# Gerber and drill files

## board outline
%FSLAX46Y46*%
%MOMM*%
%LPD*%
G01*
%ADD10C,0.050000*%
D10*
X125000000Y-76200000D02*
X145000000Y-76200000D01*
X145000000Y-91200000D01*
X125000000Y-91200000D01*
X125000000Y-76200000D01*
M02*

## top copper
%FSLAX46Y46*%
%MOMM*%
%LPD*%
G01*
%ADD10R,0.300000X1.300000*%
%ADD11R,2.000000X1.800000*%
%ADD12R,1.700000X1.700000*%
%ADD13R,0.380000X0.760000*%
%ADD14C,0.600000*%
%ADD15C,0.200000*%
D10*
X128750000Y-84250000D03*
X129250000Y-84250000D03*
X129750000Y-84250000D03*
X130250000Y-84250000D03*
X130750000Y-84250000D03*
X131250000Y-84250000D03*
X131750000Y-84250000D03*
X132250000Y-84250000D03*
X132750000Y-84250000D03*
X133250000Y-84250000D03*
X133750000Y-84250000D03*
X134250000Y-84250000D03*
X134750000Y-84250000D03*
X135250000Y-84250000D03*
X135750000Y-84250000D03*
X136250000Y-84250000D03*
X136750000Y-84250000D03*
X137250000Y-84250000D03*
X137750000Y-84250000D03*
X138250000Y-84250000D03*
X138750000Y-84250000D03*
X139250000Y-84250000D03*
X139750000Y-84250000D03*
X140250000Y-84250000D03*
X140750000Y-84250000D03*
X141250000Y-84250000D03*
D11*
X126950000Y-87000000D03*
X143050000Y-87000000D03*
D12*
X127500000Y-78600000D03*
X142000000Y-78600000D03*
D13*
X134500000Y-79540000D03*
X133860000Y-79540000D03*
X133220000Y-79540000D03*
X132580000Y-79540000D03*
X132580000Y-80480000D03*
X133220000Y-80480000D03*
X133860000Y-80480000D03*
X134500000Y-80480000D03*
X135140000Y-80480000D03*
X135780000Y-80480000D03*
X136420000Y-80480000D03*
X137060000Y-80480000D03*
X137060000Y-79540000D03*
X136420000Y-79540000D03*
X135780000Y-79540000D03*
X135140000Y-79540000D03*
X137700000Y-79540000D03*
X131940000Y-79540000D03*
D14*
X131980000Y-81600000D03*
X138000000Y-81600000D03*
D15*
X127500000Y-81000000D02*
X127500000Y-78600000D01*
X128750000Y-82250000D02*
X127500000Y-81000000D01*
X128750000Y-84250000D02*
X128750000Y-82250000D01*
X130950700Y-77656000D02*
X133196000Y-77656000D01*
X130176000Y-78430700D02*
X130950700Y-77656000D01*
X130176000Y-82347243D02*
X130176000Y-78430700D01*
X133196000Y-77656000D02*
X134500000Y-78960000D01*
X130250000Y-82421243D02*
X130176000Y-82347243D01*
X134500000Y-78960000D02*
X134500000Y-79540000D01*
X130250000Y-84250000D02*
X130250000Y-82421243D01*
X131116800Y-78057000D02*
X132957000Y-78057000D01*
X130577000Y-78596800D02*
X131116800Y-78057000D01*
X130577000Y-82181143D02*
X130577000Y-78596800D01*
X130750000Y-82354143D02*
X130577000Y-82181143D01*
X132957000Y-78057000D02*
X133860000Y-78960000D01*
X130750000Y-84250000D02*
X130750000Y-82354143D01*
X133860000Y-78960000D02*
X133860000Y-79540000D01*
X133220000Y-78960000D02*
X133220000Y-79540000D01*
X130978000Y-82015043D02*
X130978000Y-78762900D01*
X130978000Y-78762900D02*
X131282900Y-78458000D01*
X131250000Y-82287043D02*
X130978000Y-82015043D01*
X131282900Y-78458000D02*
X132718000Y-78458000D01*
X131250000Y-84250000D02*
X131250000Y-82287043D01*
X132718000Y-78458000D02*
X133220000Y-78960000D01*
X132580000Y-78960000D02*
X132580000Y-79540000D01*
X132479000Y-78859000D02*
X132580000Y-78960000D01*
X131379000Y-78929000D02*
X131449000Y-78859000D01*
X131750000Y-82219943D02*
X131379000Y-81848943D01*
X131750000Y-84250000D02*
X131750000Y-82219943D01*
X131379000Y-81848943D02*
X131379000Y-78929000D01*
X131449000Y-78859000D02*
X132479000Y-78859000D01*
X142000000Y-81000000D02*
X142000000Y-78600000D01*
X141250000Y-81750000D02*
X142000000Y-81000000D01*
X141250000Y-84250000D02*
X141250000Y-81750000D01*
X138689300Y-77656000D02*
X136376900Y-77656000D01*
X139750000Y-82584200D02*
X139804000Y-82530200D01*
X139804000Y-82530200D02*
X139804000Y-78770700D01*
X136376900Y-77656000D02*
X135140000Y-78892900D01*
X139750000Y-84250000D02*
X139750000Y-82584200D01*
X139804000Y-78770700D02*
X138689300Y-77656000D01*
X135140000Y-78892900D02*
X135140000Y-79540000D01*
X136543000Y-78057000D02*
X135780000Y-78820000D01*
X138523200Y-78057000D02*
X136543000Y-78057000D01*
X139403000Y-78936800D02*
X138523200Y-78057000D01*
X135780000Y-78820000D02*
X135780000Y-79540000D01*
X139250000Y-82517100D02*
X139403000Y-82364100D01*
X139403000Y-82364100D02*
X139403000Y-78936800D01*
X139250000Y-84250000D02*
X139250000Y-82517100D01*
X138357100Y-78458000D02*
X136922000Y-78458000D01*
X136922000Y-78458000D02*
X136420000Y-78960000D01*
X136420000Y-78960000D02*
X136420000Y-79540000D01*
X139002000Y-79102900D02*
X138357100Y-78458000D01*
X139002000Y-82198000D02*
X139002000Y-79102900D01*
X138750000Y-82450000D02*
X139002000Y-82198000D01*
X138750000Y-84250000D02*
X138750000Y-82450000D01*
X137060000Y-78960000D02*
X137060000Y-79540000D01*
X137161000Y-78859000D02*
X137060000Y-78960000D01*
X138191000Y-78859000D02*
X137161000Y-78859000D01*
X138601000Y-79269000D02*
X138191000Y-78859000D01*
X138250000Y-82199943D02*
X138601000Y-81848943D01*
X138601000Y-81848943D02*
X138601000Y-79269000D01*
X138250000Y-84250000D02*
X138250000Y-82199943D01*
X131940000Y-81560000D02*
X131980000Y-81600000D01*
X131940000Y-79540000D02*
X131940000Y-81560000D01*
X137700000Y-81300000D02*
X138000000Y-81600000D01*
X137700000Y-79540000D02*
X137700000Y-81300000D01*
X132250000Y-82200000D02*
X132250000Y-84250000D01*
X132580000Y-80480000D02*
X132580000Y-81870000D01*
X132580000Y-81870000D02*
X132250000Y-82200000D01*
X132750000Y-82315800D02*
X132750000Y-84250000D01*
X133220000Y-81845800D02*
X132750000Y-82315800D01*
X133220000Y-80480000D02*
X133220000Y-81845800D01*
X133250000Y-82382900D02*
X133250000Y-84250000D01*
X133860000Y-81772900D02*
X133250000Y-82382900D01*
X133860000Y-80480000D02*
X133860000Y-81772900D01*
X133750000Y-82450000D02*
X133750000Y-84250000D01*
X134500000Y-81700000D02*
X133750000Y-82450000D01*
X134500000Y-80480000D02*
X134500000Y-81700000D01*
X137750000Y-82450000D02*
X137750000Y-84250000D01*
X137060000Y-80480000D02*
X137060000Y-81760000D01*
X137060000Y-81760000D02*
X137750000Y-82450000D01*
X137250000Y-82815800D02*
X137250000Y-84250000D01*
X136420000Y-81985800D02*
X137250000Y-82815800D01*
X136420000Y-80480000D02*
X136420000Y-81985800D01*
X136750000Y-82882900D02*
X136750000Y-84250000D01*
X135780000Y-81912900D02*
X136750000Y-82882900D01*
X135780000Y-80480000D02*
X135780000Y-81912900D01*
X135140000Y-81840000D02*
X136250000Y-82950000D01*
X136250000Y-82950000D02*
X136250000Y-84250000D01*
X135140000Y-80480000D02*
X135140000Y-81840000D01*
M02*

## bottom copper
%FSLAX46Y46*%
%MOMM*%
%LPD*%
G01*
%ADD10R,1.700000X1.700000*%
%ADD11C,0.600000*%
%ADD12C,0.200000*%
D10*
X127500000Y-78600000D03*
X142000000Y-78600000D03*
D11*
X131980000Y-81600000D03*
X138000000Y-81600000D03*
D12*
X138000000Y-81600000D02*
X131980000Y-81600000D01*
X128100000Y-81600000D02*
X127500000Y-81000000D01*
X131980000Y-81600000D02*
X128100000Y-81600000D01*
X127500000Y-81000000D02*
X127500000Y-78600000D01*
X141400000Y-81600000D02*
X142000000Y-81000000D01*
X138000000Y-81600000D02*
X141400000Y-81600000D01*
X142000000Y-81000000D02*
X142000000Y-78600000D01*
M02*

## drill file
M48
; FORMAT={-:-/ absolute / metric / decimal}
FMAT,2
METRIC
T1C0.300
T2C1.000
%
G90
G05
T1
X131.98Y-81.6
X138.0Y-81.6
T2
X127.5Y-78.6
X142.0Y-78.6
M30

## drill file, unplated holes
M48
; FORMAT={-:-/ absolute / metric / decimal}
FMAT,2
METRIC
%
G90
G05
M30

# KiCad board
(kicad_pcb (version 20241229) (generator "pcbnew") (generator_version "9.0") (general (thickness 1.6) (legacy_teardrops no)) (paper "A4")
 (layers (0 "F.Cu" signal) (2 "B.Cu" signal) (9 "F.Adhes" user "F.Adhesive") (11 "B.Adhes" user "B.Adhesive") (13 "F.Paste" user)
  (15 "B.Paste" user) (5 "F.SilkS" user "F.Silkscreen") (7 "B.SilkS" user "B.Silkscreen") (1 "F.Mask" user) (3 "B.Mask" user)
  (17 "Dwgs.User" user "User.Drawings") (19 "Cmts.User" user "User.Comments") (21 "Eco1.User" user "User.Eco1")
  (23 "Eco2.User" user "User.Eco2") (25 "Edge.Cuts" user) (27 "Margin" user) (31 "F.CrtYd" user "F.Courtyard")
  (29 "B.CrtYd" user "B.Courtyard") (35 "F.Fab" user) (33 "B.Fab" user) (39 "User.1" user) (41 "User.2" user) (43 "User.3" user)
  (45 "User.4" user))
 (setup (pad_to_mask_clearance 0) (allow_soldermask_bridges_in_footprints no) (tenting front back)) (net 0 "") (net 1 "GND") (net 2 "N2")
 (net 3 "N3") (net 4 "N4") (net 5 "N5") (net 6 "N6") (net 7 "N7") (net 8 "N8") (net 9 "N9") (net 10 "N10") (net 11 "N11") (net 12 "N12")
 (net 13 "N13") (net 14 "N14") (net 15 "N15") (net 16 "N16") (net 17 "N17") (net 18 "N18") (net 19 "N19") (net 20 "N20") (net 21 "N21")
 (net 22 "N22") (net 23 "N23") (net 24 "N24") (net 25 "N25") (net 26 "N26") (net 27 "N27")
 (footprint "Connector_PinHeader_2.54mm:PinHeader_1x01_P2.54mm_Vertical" (layer "F.Cu") (at 127.5 78.6)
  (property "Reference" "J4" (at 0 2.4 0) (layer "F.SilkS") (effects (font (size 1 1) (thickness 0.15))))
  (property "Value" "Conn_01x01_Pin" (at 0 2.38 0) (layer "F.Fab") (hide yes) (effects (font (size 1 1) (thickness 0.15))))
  (pad "1" thru_hole rect (at 0 0) (size 1.7 1.7) (drill 1) (layers "*.Cu" "*.Mask") (remove_unused_layers no) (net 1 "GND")))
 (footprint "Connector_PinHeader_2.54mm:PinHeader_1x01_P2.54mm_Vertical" (layer "F.Cu") (at 142 78.6)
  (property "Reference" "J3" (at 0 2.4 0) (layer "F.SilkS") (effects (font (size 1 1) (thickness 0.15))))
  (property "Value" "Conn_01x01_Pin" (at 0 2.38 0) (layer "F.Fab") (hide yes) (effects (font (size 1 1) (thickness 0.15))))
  (pad "1" thru_hole rect (at 0 0) (size 1.7 1.7) (drill 1) (layers "*.Cu" "*.Mask") (remove_unused_layers no) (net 1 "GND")))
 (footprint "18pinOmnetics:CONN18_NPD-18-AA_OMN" (layer "F.Cu") (at 134.5 78.6 180)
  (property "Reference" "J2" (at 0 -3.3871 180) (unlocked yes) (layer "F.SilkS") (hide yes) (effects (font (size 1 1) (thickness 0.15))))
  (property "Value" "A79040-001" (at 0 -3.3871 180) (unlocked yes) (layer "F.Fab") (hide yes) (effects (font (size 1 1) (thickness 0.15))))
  (pad "0" smd rect (at 0 -0.94 180) (size 0.38 0.76) (layers "F.Cu" "F.Mask" "F.Paste") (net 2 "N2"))
  (pad "1" smd rect (at 0.64 -0.94 180) (size 0.38 0.76) (layers "F.Cu" "F.Mask" "F.Paste") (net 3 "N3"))
  (pad "2" smd rect (at 1.28 -0.94 180) (size 0.38 0.76) (layers "F.Cu" "F.Mask" "F.Paste") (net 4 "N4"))
  (pad "3" smd rect (at 1.92 -0.94 180) (size 0.38 0.76) (layers "F.Cu" "F.Mask" "F.Paste") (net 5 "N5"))
  (pad "4" smd rect (at 1.92 -1.88 180) (size 0.38 0.76) (layers "F.Cu" "F.Mask" "F.Paste") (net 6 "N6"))
  (pad "5" smd rect (at 1.28 -1.88 180) (size 0.38 0.76) (layers "F.Cu" "F.Mask" "F.Paste") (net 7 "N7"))
  (pad "6" smd rect (at 0.64 -1.88 180) (size 0.38 0.76) (layers "F.Cu" "F.Mask" "F.Paste") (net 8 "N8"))
  (pad "7" smd rect (at 0 -1.88 180) (size 0.38 0.76) (layers "F.Cu" "F.Mask" "F.Paste") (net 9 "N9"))
  (pad "8" smd rect (at -0.64 -1.88 180) (size 0.38 0.76) (layers "F.Cu" "F.Mask" "F.Paste") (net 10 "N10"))
  (pad "9" smd rect (at -1.28 -1.88 180) (size 0.38 0.76) (layers "F.Cu" "F.Mask" "F.Paste") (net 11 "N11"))
  (pad "10" smd rect (at -1.92 -1.88 180) (size 0.38 0.76) (layers "F.Cu" "F.Mask" "F.Paste") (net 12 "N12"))
  (pad "11" smd rect (at -2.56 -1.88 180) (size 0.38 0.76) (layers "F.Cu" "F.Mask" "F.Paste") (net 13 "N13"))
  (pad "12" smd rect (at -2.56 -0.94 180) (size 0.38 0.76) (layers "F.Cu" "F.Mask" "F.Paste") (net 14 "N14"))
  (pad "13" smd rect (at -1.92 -0.94 180) (size 0.38 0.76) (layers "F.Cu" "F.Mask" "F.Paste") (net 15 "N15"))
  (pad "14" smd rect (at -1.28 -0.94 180) (size 0.38 0.76) (layers "F.Cu" "F.Mask" "F.Paste") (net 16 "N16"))
  (pad "15" smd rect (at -0.64 -0.94 180) (size 0.38 0.76) (layers "F.Cu" "F.Mask" "F.Paste") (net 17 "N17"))
  (pad "16" smd rect (at -3.2 -0.94 180) (size 0.38 0.76) (layers "F.Cu" "F.Mask" "F.Paste") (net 1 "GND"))
  (pad "17" smd rect (at 2.56 -0.94 180) (size 0.38 0.76) (layers "F.Cu" "F.Mask" "F.Paste") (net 1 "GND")))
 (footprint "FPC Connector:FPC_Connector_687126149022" (layer "F.Cu") (at 135 87.6)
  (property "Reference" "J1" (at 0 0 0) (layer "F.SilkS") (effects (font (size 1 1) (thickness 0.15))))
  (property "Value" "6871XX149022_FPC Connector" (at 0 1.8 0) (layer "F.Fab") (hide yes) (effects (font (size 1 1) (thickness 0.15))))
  (pad "1" smd rect (at -6.25 -3.35) (size 0.3 1.3) (layers "F.Cu" "F.Mask" "F.Paste") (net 1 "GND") (solder_mask_margin 0.102))
  (pad "2" smd rect (at -5.75 -3.35) (size 0.3 1.3) (layers "F.Cu" "F.Mask" "F.Paste") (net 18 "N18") (solder_mask_margin 0.102))
  (pad "3" smd rect (at -5.25 -3.35) (size 0.3 1.3) (layers "F.Cu" "F.Mask" "F.Paste") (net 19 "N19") (solder_mask_margin 0.102))
  (pad "4" smd rect (at -4.75 -3.35) (size 0.3 1.3) (layers "F.Cu" "F.Mask" "F.Paste") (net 2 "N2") (solder_mask_margin 0.102))
  (pad "5" smd rect (at -4.25 -3.35) (size 0.3 1.3) (layers "F.Cu" "F.Mask" "F.Paste") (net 3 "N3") (solder_mask_margin 0.102))
  (pad "6" smd rect (at -3.75 -3.35) (size 0.3 1.3) (layers "F.Cu" "F.Mask" "F.Paste") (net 4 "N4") (solder_mask_margin 0.102))
  (pad "7" smd rect (at -3.25 -3.35) (size 0.3 1.3) (layers "F.Cu" "F.Mask" "F.Paste") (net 5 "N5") (solder_mask_margin 0.102))
  (pad "8" smd rect (at -2.75 -3.35) (size 0.3 1.3) (layers "F.Cu" "F.Mask" "F.Paste") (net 6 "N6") (solder_mask_margin 0.102))
  (pad "9" smd rect (at -2.25 -3.35) (size 0.3 1.3) (layers "F.Cu" "F.Mask" "F.Paste") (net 7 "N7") (solder_mask_margin 0.102))
  (pad "10" smd rect (at -1.75 -3.35) (size 0.3 1.3) (layers "F.Cu" "F.Mask" "F.Paste") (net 8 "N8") (solder_mask_margin 0.102))
  (pad "11" smd rect (at -1.25 -3.35) (size 0.3 1.3) (layers "F.Cu" "F.Mask" "F.Paste") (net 9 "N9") (solder_mask_margin 0.102))
  (pad "12" smd rect (at -0.75 -3.35) (size 0.3 1.3) (layers "F.Cu" "F.Mask" "F.Paste") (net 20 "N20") (solder_mask_margin 0.102))
  (pad "13" smd rect (at -0.25 -3.35) (size 0.3 1.3) (layers "F.Cu" "F.Mask" "F.Paste") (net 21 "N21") (solder_mask_margin 0.102))
  (pad "14" smd rect (at 0.25 -3.35) (size 0.3 1.3) (layers "F.Cu" "F.Mask" "F.Paste") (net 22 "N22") (solder_mask_margin 0.102))
  (pad "15" smd rect (at 0.75 -3.35) (size 0.3 1.3) (layers "F.Cu" "F.Mask" "F.Paste") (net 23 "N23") (solder_mask_margin 0.102))
  (pad "16" smd rect (at 1.25 -3.35) (size 0.3 1.3) (layers "F.Cu" "F.Mask" "F.Paste") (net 10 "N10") (solder_mask_margin 0.102))
  (pad "17" smd rect (at 1.75 -3.35) (size 0.3 1.3) (layers "F.Cu" "F.Mask" "F.Paste") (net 11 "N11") (solder_mask_margin 0.102))
  (pad "18" smd rect (at 2.25 -3.35) (size 0.3 1.3) (layers "F.Cu" "F.Mask" "F.Paste") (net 12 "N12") (solder_mask_margin 0.102))
  (pad "19" smd rect (at 2.75 -3.35) (size 0.3 1.3) (layers "F.Cu" "F.Mask" "F.Paste") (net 13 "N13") (solder_mask_margin 0.102))
  (pad "20" smd rect (at 3.25 -3.35) (size 0.3 1.3) (layers "F.Cu" "F.Mask" "F.Paste") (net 14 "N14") (solder_mask_margin 0.102))
  (pad "21" smd rect (at 3.75 -3.35) (size 0.3 1.3) (layers "F.Cu" "F.Mask" "F.Paste") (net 15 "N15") (solder_mask_margin 0.102))
  (pad "22" smd rect (at 4.25 -3.35) (size 0.3 1.3) (layers "F.Cu" "F.Mask" "F.Paste") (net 16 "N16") (solder_mask_margin 0.102))
  (pad "23" smd rect (at 4.75 -3.35) (size 0.3 1.3) (layers "F.Cu" "F.Mask" "F.Paste") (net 17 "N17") (solder_mask_margin 0.102))
  (pad "24" smd rect (at 5.25 -3.35) (size 0.3 1.3) (layers "F.Cu" "F.Mask" "F.Paste") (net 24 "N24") (solder_mask_margin 0.102))
  (pad "25" smd rect (at 5.75 -3.35) (size 0.3 1.3) (layers "F.Cu" "F.Mask" "F.Paste") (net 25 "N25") (solder_mask_margin 0.102))
  (pad "26" smd rect (at 6.25 -3.35) (size 0.3 1.3) (layers "F.Cu" "F.Mask" "F.Paste") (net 1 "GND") (solder_mask_margin 0.102))
  (pad "Z1" smd rect (at -8.05 -0.6) (size 2 1.8) (layers "F.Cu" "F.Mask" "F.Paste") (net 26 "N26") (solder_mask_margin 0.102))
  (pad "Z2" smd rect (at 8.05 -0.6) (size 2 1.8) (layers "F.Cu" "F.Mask" "F.Paste") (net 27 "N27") (solder_mask_margin 0.102)))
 (gr_rect (start 125 76.2) (end 145 91.2) (stroke (width 0.05) (type default)) (fill no) (layer "Edge.Cuts"))
 (segment (start 136.25 82.95) (end 136.25 84.25) (width 0.2) (layer "F.Cu") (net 10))
 (segment (start 135.14 81.84) (end 136.25 82.95) (width 0.2) (layer "F.Cu") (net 10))
 (segment (start 135.14 80.48) (end 135.14 81.84) (width 0.2) (layer "F.Cu") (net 10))
 (segment (start 132.58 78.96) (end 132.58 79.54) (width 0.2) (layer "F.Cu") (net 5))
 (segment (start 131.379 81.848943) (end 131.379 78.929) (width 0.2) (layer "F.Cu") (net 5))
 (segment (start 131.75 82.219943) (end 131.379 81.848943) (width 0.2) (layer "F.Cu") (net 5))
 (segment (start 131.75 84.25) (end 131.75 82.219943) (width 0.2) (layer "F.Cu") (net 5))
 (segment (start 131.449 78.859) (end 132.479 78.859) (width 0.2) (layer "F.Cu") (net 5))
 (segment (start 132.479 78.859) (end 132.58 78.96) (width 0.2) (layer "F.Cu") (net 5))
 (segment (start 131.379 78.929) (end 131.449 78.859) (width 0.2) (layer "F.Cu") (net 5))
 (segment (start 133.25 82.3829) (end 133.25 84.25) (width 0.2) (layer "F.Cu") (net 8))
 (segment (start 133.86 80.48) (end 133.86 81.7729) (width 0.2) (layer "F.Cu") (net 8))
 (segment (start 133.86 81.7729) (end 133.25 82.3829) (width 0.2) (layer "F.Cu") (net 8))
 (segment (start 131.1168 78.057) (end 132.957 78.057) (width 0.2) (layer "F.Cu") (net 3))
 (segment (start 133.86 78.96) (end 133.86 79.54) (width 0.2) (layer "F.Cu") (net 3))
 (segment (start 130.75 84.25) (end 130.75 82.354143) (width 0.2) (layer "F.Cu") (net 3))
 (segment (start 130.75 82.354143) (end 130.577 82.181143) (width 0.2) (layer "F.Cu") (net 3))
 (segment (start 130.577 82.181143) (end 130.577 78.5968) (width 0.2) (layer "F.Cu") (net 3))
 (segment (start 132.957 78.057) (end 133.86 78.96) (width 0.2) (layer "F.Cu") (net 3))
 (segment (start 130.577 78.5968) (end 131.1168 78.057) (width 0.2) (layer "F.Cu") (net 3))
 (segment (start 139.25 84.25) (end 139.25 82.5171) (width 0.2) (layer "F.Cu") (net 16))
 (segment (start 139.403 78.9368) (end 138.5232 78.057) (width 0.2) (layer "F.Cu") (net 16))
 (segment (start 136.543 78.057) (end 135.78 78.82) (width 0.2) (layer "F.Cu") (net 16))
 (segment (start 139.403 82.3641) (end 139.403 78.9368) (width 0.2) (layer "F.Cu") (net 16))
 (segment (start 135.78 78.82) (end 135.78 79.54) (width 0.2) (layer "F.Cu") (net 16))
 (segment (start 139.25 82.5171) (end 139.403 82.3641) (width 0.2) (layer "F.Cu") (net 16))
 (segment (start 138.5232 78.057) (end 136.543 78.057) (width 0.2) (layer "F.Cu") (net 16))
 (segment (start 134.5 80.48) (end 134.5 81.7) (width 0.2) (layer "F.Cu") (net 9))
 (segment (start 133.75 82.45) (end 133.75 84.25) (width 0.2) (layer "F.Cu") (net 9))
 (segment (start 134.5 81.7) (end 133.75 82.45) (width 0.2) (layer "F.Cu") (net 9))
 (segment (start 138.75 82.45) (end 139.002 82.198) (width 0.2) (layer "F.Cu") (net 15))
 (segment (start 139.002 82.198) (end 139.002 79.1029) (width 0.2) (layer "F.Cu") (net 15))
 (segment (start 138.3571 78.458) (end 136.922 78.458) (width 0.2) (layer "F.Cu") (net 15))
 (segment (start 138.75 84.25) (end 138.75 82.45) (width 0.2) (layer "F.Cu") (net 15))
 (segment (start 139.002 79.1029) (end 138.3571 78.458) (width 0.2) (layer "F.Cu") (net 15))
 (segment (start 136.42 78.96) (end 136.42 79.54) (width 0.2) (layer "F.Cu") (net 15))
 (segment (start 136.922 78.458) (end 136.42 78.96) (width 0.2) (layer "F.Cu") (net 15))
 (segment (start 131.25 84.25) (end 131.25 82.287043) (width 0.2) (layer "F.Cu") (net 4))
 (segment (start 130.978 78.7629) (end 131.2829 78.458) (width 0.2) (layer "F.Cu") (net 4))
 (segment (start 133.22 78.96) (end 133.22 79.54) (width 0.2) (layer "F.Cu") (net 4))
 (segment (start 131.2829 78.458) (end 132.718 78.458) (width 0.2) (layer "F.Cu") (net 4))
 (segment (start 130.978 82.015043) (end 130.978 78.7629) (width 0.2) (layer "F.Cu") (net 4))
 (segment (start 132.718 78.458) (end 133.22 78.96) (width 0.2) (layer "F.Cu") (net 4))
 (segment (start 131.25 82.287043) (end 130.978 82.015043) (width 0.2) (layer "F.Cu") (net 4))
 (segment (start 135.78 80.48) (end 135.78 81.9129) (width 0.2) (layer "F.Cu") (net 11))
 (segment (start 135.78 81.9129) (end 136.75 82.8829) (width 0.2) (layer "F.Cu") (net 11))
 (segment (start 136.75 82.8829) (end 136.75 84.25) (width 0.2) (layer "F.Cu") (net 11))
 (segment (start 133.22 80.48) (end 133.22 81.8458) (width 0.2) (layer "F.Cu") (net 7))
 (segment (start 132.75 82.3158) (end 132.75 84.25) (width 0.2) (layer "F.Cu") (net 7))
 (segment (start 133.22 81.8458) (end 132.75 82.3158) (width 0.2) (layer "F.Cu") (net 7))
 (segment (start 136.42 80.48) (end 136.42 81.9858) (width 0.2) (layer "F.Cu") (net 12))
 (segment (start 136.42 81.9858) (end 137.25 82.8158) (width 0.2) (layer "F.Cu") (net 12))
 (segment (start 137.25 82.8158) (end 137.25 84.25) (width 0.2) (layer "F.Cu") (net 12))
 (segment (start 138.25 84.25) (end 138.25 82.199943) (width 0.2) (layer "F.Cu") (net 14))
 (segment (start 137.06 78.96) (end 137.06 79.54) (width 0.2) (layer "F.Cu") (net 14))
 (segment (start 138.601 79.269) (end 138.191 78.859) (width 0.2) (layer "F.Cu") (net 14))
 (segment (start 137.161 78.859) (end 137.06 78.96) (width 0.2) (layer "F.Cu") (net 14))
 (segment (start 138.25 82.199943) (end 138.601 81.848943) (width 0.2) (layer "F.Cu") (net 14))
 (segment (start 138.191 78.859) (end 137.161 78.859) (width 0.2) (layer "F.Cu") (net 14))
 (segment (start 138.601 81.848943) (end 138.601 79.269) (width 0.2) (layer "F.Cu") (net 14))
 (segment (start 131.94 81.56) (end 131.98 81.6) (width 0.2) (layer "F.Cu") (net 1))
 (segment (start 137.7 81.3) (end 138 81.6) (width 0.2) (layer "F.Cu") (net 1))
 (segment (start 127.5 81) (end 127.5 78.6) (width 0.2) (layer "F.Cu") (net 1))
 (segment (start 142 81) (end 142 78.6) (width 0.2) (layer "F.Cu") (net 1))
 (segment (start 141.25 84.25) (end 141.25 81.75) (width 0.2) (layer "F.Cu") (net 1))
 (segment (start 128.75 82.25) (end 127.5 81) (width 0.2) (layer "F.Cu") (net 1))
 (segment (start 131.94 79.54) (end 131.94 81.56) (width 0.2) (layer "F.Cu") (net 1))
 (segment (start 137.7 79.54) (end 137.7 81.3) (width 0.2) (layer "F.Cu") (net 1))
 (segment (start 141.25 81.75) (end 142 81) (width 0.2) (layer "F.Cu") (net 1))
 (segment (start 128.75 84.25) (end 128.75 82.25) (width 0.2) (layer "F.Cu") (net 1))
 (via (at 138 81.6) (size 0.6) (drill 0.3) (layers "F.Cu" "B.Cu") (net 1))
 (via (at 131.98 81.6) (size 0.6) (drill 0.3) (layers "F.Cu" "B.Cu") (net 1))
 (segment (start 128.1 81.6) (end 127.5 81) (width 0.2) (layer "B.Cu") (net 1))
 (segment (start 142 81) (end 142 78.6) (width 0.2) (layer "B.Cu") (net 1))
 (segment (start 138 81.6) (end 131.98 81.6) (width 0.2) (layer "B.Cu") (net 1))
 (segment (start 138 81.6) (end 141.4 81.6) (width 0.2) (layer "B.Cu") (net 1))
 (segment (start 141.4 81.6) (end 142 81) (width 0.2) (layer "B.Cu") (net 1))
 (segment (start 127.5 81) (end 127.5 78.6) (width 0.2) (layer "B.Cu") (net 1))
 (segment (start 131.98 81.6) (end 128.1 81.6) (width 0.2) (layer "B.Cu") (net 1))
 (segment (start 132.58 80.48) (end 132.58 81.87) (width 0.2) (layer "F.Cu") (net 6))
 (segment (start 132.58 81.87) (end 132.25 82.2) (width 0.2) (layer "F.Cu") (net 6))
 (segment (start 132.25 82.2) (end 132.25 84.25) (width 0.2) (layer "F.Cu") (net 6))
 (segment (start 130.9507 77.656) (end 133.196 77.656) (width 0.2) (layer "F.Cu") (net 2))
 (segment (start 130.176 82.347243) (end 130.176 78.4307) (width 0.2) (layer "F.Cu") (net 2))
 (segment (start 134.5 78.96) (end 134.5 79.54) (width 0.2) (layer "F.Cu") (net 2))
 (segment (start 130.176 78.4307) (end 130.9507 77.656) (width 0.2) (layer "F.Cu") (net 2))
 (segment (start 130.25 84.25) (end 130.25 82.421243) (width 0.2) (layer "F.Cu") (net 2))
 (segment (start 133.196 77.656) (end 134.5 78.96) (width 0.2) (layer "F.Cu") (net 2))
 (segment (start 130.25 82.421243) (end 130.176 82.347243) (width 0.2) (layer "F.Cu") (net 2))
 (segment (start 137.75 82.45) (end 137.75 84.25) (width 0.2) (layer "F.Cu") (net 13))
 (segment (start 137.06 80.48) (end 137.06 81.76) (width 0.2) (layer "F.Cu") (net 13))
 (segment (start 137.06 81.76) (end 137.75 82.45) (width 0.2) (layer "F.Cu") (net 13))
 (segment (start 139.804 82.5302) (end 139.804 78.7707) (width 0.2) (layer "F.Cu") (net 17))
 (segment (start 139.75 84.25) (end 139.75 82.5842) (width 0.2) (layer "F.Cu") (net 17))
 (segment (start 136.3769 77.656) (end 135.14 78.8929) (width 0.2) (layer "F.Cu") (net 17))
 (segment (start 138.6893 77.656) (end 136.3769 77.656) (width 0.2) (layer "F.Cu") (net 17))
 (segment (start 135.14 78.8929) (end 135.14 79.54) (width 0.2) (layer "F.Cu") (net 17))
 (segment (start 139.75 82.5842) (end 139.804 82.5302) (width 0.2) (layer "F.Cu") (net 17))
 (segment (start 139.804 78.7707) (end 138.6893 77.656) (width 0.2) (layer "F.Cu") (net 17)))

